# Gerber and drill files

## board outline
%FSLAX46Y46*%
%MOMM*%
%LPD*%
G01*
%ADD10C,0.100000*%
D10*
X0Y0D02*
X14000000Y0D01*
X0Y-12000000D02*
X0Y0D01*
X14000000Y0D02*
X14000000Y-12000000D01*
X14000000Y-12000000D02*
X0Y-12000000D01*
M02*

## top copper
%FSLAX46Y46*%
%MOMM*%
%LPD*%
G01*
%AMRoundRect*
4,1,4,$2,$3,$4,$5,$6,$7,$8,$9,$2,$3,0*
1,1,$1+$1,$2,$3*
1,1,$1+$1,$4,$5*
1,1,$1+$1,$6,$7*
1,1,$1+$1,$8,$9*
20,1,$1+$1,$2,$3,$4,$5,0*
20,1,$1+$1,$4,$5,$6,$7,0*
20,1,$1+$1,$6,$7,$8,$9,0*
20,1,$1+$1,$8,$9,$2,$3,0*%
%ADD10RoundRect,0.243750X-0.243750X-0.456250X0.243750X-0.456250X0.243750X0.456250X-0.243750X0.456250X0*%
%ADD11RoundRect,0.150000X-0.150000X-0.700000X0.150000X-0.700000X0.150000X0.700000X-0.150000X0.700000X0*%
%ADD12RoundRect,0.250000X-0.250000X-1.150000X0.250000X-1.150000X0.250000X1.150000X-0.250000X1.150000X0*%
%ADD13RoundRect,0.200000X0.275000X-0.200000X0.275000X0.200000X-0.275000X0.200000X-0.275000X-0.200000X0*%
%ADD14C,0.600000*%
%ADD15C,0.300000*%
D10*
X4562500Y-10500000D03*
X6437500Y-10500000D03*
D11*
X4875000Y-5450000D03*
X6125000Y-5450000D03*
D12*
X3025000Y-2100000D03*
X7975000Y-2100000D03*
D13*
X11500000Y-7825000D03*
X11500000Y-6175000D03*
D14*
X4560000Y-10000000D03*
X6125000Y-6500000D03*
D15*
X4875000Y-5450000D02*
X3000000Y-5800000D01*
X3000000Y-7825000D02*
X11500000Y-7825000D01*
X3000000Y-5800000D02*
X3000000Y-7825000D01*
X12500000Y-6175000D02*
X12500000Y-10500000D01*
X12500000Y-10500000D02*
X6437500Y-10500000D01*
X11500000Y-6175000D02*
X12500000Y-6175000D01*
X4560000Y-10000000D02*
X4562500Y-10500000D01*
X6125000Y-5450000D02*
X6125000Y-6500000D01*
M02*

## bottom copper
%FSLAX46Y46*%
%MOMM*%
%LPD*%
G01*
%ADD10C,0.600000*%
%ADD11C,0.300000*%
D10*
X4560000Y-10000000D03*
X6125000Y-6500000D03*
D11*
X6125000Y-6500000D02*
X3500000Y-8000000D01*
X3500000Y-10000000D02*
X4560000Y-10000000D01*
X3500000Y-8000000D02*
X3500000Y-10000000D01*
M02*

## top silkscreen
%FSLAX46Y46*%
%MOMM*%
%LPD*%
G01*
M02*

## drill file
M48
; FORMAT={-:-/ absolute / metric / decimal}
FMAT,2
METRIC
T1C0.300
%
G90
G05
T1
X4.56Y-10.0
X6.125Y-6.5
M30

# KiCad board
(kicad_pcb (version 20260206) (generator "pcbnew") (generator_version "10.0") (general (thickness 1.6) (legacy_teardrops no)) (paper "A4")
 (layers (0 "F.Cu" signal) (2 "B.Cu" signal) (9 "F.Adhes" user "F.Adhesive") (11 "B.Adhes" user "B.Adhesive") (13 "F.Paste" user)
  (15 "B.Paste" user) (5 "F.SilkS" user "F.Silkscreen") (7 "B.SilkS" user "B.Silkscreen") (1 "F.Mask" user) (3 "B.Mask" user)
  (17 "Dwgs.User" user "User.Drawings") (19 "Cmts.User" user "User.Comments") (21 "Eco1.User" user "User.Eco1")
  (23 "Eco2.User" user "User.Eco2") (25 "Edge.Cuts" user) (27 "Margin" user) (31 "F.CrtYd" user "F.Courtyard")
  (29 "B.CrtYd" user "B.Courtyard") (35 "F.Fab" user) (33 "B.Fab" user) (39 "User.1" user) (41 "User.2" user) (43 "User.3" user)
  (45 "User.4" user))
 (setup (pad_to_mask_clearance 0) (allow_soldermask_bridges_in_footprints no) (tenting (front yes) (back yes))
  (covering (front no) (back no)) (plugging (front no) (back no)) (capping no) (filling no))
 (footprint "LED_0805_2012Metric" (layer "F.Cu") (at 5.5 10.5)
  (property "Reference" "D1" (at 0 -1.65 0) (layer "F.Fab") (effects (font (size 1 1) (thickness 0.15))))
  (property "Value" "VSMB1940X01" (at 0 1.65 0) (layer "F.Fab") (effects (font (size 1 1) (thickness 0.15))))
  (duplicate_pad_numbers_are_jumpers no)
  (pad "1" smd roundrect (at -0.9375 0) (size 0.975 1.4) (layers "F.Cu" "F.Mask" "F.Paste") (roundrect_rratio 0.25) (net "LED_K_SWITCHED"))
  (pad "2" smd roundrect (at 0.9375 0) (size 0.975 1.4) (layers "F.Cu" "F.Mask" "F.Paste") (roundrect_rratio 0.25) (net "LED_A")))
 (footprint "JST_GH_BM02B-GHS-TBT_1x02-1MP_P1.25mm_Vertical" (layer "F.Cu") (at 5.5 3.5)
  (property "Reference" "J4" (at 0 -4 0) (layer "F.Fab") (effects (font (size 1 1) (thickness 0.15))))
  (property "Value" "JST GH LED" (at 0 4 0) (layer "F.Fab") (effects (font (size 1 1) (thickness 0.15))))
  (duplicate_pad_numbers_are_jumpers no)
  (pad "1" smd roundrect (at -0.625 1.95) (size 0.6 1.7) (layers "F.Cu" "F.Mask" "F.Paste") (roundrect_rratio 0.25) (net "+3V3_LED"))
  (pad "2" smd roundrect (at 0.625 1.95) (size 0.6 1.7) (layers "F.Cu" "F.Mask" "F.Paste") (roundrect_rratio 0.25) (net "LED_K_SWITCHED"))
  (pad "MP" smd roundrect (at -2.475 -1.4) (size 1 2.8) (layers "F.Cu" "F.Mask" "F.Paste") (roundrect_rratio 0.25))
  (pad "MP" smd roundrect (at 2.475 -1.4) (size 1 2.8) (layers "F.Cu" "F.Mask" "F.Paste") (roundrect_rratio 0.25)))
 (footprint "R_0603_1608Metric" (layer "F.Cu") (at 11.5 7 90)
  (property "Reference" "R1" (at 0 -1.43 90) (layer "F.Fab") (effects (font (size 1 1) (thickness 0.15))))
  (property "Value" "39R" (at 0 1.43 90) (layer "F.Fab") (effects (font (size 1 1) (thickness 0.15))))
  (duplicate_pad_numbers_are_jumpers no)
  (pad "1" smd roundrect (at -0.825 0 90) (size 0.8 0.95) (layers "F.Cu" "F.Mask" "F.Paste") (roundrect_rratio 0.25) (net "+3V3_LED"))
  (pad "2" smd roundrect (at 0.825 0 90) (size 0.8 0.95) (layers "F.Cu" "F.Mask" "F.Paste") (roundrect_rratio 0.25) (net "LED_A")))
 (gr_line (start 0 0) (end 14 0) (stroke (width 0.1) (type default)) (layer "Edge.Cuts"))
 (gr_line (start 0 12) (end 0 0) (stroke (width 0.1) (type default)) (layer "Edge.Cuts"))
 (gr_line (start 14 0) (end 14 12) (stroke (width 0.1) (type default)) (layer "Edge.Cuts"))
 (gr_line (start 14 12) (end 0 12) (stroke (width 0.1) (type default)) (layer "Edge.Cuts"))
 (segment (start 4.875 5.45) (end 3 5.8) (width 0.3) (layer "F.Cu") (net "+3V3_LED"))
 (segment (start 3 7.825) (end 11.5 7.825) (width 0.3) (layer "F.Cu") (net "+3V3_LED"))
 (segment (start 3 5.8) (end 3 7.825) (width 0.3) (layer "F.Cu") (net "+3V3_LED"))
 (segment (start 12.5 6.175) (end 12.5 10.5) (width 0.3) (layer "F.Cu") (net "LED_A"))
 (segment (start 12.5 10.5) (end 6.4375 10.5) (width 0.3) (layer "F.Cu") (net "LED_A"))
 (segment (start 11.5 6.175) (end 12.5 6.175) (width 0.3) (layer "F.Cu") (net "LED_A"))
 (segment (start 4.56 10) (end 4.5625 10.5) (width 0.3) (layer "F.Cu") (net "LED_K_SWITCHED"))
 (segment (start 6.125 5.45) (end 6.125 6.5) (width 0.3) (layer "F.Cu") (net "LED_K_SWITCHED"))
 (via (at 4.56 10) (size 0.6) (drill 0.3) (layers "F.Cu" "B.Cu") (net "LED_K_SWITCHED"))
 (via (at 6.125 6.5) (size 0.6) (drill 0.3) (layers "F.Cu" "B.Cu") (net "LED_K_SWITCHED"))
 (segment (start 6.125 6.5) (end 3.5 8) (width 0.3) (layer "B.Cu") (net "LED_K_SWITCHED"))
 (segment (start 3.5 10) (end 4.56 10) (width 0.3) (layer "B.Cu") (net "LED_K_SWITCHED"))
 (segment (start 3.5 8) (end 3.5 10) (width 0.3) (layer "B.Cu") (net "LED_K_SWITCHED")))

